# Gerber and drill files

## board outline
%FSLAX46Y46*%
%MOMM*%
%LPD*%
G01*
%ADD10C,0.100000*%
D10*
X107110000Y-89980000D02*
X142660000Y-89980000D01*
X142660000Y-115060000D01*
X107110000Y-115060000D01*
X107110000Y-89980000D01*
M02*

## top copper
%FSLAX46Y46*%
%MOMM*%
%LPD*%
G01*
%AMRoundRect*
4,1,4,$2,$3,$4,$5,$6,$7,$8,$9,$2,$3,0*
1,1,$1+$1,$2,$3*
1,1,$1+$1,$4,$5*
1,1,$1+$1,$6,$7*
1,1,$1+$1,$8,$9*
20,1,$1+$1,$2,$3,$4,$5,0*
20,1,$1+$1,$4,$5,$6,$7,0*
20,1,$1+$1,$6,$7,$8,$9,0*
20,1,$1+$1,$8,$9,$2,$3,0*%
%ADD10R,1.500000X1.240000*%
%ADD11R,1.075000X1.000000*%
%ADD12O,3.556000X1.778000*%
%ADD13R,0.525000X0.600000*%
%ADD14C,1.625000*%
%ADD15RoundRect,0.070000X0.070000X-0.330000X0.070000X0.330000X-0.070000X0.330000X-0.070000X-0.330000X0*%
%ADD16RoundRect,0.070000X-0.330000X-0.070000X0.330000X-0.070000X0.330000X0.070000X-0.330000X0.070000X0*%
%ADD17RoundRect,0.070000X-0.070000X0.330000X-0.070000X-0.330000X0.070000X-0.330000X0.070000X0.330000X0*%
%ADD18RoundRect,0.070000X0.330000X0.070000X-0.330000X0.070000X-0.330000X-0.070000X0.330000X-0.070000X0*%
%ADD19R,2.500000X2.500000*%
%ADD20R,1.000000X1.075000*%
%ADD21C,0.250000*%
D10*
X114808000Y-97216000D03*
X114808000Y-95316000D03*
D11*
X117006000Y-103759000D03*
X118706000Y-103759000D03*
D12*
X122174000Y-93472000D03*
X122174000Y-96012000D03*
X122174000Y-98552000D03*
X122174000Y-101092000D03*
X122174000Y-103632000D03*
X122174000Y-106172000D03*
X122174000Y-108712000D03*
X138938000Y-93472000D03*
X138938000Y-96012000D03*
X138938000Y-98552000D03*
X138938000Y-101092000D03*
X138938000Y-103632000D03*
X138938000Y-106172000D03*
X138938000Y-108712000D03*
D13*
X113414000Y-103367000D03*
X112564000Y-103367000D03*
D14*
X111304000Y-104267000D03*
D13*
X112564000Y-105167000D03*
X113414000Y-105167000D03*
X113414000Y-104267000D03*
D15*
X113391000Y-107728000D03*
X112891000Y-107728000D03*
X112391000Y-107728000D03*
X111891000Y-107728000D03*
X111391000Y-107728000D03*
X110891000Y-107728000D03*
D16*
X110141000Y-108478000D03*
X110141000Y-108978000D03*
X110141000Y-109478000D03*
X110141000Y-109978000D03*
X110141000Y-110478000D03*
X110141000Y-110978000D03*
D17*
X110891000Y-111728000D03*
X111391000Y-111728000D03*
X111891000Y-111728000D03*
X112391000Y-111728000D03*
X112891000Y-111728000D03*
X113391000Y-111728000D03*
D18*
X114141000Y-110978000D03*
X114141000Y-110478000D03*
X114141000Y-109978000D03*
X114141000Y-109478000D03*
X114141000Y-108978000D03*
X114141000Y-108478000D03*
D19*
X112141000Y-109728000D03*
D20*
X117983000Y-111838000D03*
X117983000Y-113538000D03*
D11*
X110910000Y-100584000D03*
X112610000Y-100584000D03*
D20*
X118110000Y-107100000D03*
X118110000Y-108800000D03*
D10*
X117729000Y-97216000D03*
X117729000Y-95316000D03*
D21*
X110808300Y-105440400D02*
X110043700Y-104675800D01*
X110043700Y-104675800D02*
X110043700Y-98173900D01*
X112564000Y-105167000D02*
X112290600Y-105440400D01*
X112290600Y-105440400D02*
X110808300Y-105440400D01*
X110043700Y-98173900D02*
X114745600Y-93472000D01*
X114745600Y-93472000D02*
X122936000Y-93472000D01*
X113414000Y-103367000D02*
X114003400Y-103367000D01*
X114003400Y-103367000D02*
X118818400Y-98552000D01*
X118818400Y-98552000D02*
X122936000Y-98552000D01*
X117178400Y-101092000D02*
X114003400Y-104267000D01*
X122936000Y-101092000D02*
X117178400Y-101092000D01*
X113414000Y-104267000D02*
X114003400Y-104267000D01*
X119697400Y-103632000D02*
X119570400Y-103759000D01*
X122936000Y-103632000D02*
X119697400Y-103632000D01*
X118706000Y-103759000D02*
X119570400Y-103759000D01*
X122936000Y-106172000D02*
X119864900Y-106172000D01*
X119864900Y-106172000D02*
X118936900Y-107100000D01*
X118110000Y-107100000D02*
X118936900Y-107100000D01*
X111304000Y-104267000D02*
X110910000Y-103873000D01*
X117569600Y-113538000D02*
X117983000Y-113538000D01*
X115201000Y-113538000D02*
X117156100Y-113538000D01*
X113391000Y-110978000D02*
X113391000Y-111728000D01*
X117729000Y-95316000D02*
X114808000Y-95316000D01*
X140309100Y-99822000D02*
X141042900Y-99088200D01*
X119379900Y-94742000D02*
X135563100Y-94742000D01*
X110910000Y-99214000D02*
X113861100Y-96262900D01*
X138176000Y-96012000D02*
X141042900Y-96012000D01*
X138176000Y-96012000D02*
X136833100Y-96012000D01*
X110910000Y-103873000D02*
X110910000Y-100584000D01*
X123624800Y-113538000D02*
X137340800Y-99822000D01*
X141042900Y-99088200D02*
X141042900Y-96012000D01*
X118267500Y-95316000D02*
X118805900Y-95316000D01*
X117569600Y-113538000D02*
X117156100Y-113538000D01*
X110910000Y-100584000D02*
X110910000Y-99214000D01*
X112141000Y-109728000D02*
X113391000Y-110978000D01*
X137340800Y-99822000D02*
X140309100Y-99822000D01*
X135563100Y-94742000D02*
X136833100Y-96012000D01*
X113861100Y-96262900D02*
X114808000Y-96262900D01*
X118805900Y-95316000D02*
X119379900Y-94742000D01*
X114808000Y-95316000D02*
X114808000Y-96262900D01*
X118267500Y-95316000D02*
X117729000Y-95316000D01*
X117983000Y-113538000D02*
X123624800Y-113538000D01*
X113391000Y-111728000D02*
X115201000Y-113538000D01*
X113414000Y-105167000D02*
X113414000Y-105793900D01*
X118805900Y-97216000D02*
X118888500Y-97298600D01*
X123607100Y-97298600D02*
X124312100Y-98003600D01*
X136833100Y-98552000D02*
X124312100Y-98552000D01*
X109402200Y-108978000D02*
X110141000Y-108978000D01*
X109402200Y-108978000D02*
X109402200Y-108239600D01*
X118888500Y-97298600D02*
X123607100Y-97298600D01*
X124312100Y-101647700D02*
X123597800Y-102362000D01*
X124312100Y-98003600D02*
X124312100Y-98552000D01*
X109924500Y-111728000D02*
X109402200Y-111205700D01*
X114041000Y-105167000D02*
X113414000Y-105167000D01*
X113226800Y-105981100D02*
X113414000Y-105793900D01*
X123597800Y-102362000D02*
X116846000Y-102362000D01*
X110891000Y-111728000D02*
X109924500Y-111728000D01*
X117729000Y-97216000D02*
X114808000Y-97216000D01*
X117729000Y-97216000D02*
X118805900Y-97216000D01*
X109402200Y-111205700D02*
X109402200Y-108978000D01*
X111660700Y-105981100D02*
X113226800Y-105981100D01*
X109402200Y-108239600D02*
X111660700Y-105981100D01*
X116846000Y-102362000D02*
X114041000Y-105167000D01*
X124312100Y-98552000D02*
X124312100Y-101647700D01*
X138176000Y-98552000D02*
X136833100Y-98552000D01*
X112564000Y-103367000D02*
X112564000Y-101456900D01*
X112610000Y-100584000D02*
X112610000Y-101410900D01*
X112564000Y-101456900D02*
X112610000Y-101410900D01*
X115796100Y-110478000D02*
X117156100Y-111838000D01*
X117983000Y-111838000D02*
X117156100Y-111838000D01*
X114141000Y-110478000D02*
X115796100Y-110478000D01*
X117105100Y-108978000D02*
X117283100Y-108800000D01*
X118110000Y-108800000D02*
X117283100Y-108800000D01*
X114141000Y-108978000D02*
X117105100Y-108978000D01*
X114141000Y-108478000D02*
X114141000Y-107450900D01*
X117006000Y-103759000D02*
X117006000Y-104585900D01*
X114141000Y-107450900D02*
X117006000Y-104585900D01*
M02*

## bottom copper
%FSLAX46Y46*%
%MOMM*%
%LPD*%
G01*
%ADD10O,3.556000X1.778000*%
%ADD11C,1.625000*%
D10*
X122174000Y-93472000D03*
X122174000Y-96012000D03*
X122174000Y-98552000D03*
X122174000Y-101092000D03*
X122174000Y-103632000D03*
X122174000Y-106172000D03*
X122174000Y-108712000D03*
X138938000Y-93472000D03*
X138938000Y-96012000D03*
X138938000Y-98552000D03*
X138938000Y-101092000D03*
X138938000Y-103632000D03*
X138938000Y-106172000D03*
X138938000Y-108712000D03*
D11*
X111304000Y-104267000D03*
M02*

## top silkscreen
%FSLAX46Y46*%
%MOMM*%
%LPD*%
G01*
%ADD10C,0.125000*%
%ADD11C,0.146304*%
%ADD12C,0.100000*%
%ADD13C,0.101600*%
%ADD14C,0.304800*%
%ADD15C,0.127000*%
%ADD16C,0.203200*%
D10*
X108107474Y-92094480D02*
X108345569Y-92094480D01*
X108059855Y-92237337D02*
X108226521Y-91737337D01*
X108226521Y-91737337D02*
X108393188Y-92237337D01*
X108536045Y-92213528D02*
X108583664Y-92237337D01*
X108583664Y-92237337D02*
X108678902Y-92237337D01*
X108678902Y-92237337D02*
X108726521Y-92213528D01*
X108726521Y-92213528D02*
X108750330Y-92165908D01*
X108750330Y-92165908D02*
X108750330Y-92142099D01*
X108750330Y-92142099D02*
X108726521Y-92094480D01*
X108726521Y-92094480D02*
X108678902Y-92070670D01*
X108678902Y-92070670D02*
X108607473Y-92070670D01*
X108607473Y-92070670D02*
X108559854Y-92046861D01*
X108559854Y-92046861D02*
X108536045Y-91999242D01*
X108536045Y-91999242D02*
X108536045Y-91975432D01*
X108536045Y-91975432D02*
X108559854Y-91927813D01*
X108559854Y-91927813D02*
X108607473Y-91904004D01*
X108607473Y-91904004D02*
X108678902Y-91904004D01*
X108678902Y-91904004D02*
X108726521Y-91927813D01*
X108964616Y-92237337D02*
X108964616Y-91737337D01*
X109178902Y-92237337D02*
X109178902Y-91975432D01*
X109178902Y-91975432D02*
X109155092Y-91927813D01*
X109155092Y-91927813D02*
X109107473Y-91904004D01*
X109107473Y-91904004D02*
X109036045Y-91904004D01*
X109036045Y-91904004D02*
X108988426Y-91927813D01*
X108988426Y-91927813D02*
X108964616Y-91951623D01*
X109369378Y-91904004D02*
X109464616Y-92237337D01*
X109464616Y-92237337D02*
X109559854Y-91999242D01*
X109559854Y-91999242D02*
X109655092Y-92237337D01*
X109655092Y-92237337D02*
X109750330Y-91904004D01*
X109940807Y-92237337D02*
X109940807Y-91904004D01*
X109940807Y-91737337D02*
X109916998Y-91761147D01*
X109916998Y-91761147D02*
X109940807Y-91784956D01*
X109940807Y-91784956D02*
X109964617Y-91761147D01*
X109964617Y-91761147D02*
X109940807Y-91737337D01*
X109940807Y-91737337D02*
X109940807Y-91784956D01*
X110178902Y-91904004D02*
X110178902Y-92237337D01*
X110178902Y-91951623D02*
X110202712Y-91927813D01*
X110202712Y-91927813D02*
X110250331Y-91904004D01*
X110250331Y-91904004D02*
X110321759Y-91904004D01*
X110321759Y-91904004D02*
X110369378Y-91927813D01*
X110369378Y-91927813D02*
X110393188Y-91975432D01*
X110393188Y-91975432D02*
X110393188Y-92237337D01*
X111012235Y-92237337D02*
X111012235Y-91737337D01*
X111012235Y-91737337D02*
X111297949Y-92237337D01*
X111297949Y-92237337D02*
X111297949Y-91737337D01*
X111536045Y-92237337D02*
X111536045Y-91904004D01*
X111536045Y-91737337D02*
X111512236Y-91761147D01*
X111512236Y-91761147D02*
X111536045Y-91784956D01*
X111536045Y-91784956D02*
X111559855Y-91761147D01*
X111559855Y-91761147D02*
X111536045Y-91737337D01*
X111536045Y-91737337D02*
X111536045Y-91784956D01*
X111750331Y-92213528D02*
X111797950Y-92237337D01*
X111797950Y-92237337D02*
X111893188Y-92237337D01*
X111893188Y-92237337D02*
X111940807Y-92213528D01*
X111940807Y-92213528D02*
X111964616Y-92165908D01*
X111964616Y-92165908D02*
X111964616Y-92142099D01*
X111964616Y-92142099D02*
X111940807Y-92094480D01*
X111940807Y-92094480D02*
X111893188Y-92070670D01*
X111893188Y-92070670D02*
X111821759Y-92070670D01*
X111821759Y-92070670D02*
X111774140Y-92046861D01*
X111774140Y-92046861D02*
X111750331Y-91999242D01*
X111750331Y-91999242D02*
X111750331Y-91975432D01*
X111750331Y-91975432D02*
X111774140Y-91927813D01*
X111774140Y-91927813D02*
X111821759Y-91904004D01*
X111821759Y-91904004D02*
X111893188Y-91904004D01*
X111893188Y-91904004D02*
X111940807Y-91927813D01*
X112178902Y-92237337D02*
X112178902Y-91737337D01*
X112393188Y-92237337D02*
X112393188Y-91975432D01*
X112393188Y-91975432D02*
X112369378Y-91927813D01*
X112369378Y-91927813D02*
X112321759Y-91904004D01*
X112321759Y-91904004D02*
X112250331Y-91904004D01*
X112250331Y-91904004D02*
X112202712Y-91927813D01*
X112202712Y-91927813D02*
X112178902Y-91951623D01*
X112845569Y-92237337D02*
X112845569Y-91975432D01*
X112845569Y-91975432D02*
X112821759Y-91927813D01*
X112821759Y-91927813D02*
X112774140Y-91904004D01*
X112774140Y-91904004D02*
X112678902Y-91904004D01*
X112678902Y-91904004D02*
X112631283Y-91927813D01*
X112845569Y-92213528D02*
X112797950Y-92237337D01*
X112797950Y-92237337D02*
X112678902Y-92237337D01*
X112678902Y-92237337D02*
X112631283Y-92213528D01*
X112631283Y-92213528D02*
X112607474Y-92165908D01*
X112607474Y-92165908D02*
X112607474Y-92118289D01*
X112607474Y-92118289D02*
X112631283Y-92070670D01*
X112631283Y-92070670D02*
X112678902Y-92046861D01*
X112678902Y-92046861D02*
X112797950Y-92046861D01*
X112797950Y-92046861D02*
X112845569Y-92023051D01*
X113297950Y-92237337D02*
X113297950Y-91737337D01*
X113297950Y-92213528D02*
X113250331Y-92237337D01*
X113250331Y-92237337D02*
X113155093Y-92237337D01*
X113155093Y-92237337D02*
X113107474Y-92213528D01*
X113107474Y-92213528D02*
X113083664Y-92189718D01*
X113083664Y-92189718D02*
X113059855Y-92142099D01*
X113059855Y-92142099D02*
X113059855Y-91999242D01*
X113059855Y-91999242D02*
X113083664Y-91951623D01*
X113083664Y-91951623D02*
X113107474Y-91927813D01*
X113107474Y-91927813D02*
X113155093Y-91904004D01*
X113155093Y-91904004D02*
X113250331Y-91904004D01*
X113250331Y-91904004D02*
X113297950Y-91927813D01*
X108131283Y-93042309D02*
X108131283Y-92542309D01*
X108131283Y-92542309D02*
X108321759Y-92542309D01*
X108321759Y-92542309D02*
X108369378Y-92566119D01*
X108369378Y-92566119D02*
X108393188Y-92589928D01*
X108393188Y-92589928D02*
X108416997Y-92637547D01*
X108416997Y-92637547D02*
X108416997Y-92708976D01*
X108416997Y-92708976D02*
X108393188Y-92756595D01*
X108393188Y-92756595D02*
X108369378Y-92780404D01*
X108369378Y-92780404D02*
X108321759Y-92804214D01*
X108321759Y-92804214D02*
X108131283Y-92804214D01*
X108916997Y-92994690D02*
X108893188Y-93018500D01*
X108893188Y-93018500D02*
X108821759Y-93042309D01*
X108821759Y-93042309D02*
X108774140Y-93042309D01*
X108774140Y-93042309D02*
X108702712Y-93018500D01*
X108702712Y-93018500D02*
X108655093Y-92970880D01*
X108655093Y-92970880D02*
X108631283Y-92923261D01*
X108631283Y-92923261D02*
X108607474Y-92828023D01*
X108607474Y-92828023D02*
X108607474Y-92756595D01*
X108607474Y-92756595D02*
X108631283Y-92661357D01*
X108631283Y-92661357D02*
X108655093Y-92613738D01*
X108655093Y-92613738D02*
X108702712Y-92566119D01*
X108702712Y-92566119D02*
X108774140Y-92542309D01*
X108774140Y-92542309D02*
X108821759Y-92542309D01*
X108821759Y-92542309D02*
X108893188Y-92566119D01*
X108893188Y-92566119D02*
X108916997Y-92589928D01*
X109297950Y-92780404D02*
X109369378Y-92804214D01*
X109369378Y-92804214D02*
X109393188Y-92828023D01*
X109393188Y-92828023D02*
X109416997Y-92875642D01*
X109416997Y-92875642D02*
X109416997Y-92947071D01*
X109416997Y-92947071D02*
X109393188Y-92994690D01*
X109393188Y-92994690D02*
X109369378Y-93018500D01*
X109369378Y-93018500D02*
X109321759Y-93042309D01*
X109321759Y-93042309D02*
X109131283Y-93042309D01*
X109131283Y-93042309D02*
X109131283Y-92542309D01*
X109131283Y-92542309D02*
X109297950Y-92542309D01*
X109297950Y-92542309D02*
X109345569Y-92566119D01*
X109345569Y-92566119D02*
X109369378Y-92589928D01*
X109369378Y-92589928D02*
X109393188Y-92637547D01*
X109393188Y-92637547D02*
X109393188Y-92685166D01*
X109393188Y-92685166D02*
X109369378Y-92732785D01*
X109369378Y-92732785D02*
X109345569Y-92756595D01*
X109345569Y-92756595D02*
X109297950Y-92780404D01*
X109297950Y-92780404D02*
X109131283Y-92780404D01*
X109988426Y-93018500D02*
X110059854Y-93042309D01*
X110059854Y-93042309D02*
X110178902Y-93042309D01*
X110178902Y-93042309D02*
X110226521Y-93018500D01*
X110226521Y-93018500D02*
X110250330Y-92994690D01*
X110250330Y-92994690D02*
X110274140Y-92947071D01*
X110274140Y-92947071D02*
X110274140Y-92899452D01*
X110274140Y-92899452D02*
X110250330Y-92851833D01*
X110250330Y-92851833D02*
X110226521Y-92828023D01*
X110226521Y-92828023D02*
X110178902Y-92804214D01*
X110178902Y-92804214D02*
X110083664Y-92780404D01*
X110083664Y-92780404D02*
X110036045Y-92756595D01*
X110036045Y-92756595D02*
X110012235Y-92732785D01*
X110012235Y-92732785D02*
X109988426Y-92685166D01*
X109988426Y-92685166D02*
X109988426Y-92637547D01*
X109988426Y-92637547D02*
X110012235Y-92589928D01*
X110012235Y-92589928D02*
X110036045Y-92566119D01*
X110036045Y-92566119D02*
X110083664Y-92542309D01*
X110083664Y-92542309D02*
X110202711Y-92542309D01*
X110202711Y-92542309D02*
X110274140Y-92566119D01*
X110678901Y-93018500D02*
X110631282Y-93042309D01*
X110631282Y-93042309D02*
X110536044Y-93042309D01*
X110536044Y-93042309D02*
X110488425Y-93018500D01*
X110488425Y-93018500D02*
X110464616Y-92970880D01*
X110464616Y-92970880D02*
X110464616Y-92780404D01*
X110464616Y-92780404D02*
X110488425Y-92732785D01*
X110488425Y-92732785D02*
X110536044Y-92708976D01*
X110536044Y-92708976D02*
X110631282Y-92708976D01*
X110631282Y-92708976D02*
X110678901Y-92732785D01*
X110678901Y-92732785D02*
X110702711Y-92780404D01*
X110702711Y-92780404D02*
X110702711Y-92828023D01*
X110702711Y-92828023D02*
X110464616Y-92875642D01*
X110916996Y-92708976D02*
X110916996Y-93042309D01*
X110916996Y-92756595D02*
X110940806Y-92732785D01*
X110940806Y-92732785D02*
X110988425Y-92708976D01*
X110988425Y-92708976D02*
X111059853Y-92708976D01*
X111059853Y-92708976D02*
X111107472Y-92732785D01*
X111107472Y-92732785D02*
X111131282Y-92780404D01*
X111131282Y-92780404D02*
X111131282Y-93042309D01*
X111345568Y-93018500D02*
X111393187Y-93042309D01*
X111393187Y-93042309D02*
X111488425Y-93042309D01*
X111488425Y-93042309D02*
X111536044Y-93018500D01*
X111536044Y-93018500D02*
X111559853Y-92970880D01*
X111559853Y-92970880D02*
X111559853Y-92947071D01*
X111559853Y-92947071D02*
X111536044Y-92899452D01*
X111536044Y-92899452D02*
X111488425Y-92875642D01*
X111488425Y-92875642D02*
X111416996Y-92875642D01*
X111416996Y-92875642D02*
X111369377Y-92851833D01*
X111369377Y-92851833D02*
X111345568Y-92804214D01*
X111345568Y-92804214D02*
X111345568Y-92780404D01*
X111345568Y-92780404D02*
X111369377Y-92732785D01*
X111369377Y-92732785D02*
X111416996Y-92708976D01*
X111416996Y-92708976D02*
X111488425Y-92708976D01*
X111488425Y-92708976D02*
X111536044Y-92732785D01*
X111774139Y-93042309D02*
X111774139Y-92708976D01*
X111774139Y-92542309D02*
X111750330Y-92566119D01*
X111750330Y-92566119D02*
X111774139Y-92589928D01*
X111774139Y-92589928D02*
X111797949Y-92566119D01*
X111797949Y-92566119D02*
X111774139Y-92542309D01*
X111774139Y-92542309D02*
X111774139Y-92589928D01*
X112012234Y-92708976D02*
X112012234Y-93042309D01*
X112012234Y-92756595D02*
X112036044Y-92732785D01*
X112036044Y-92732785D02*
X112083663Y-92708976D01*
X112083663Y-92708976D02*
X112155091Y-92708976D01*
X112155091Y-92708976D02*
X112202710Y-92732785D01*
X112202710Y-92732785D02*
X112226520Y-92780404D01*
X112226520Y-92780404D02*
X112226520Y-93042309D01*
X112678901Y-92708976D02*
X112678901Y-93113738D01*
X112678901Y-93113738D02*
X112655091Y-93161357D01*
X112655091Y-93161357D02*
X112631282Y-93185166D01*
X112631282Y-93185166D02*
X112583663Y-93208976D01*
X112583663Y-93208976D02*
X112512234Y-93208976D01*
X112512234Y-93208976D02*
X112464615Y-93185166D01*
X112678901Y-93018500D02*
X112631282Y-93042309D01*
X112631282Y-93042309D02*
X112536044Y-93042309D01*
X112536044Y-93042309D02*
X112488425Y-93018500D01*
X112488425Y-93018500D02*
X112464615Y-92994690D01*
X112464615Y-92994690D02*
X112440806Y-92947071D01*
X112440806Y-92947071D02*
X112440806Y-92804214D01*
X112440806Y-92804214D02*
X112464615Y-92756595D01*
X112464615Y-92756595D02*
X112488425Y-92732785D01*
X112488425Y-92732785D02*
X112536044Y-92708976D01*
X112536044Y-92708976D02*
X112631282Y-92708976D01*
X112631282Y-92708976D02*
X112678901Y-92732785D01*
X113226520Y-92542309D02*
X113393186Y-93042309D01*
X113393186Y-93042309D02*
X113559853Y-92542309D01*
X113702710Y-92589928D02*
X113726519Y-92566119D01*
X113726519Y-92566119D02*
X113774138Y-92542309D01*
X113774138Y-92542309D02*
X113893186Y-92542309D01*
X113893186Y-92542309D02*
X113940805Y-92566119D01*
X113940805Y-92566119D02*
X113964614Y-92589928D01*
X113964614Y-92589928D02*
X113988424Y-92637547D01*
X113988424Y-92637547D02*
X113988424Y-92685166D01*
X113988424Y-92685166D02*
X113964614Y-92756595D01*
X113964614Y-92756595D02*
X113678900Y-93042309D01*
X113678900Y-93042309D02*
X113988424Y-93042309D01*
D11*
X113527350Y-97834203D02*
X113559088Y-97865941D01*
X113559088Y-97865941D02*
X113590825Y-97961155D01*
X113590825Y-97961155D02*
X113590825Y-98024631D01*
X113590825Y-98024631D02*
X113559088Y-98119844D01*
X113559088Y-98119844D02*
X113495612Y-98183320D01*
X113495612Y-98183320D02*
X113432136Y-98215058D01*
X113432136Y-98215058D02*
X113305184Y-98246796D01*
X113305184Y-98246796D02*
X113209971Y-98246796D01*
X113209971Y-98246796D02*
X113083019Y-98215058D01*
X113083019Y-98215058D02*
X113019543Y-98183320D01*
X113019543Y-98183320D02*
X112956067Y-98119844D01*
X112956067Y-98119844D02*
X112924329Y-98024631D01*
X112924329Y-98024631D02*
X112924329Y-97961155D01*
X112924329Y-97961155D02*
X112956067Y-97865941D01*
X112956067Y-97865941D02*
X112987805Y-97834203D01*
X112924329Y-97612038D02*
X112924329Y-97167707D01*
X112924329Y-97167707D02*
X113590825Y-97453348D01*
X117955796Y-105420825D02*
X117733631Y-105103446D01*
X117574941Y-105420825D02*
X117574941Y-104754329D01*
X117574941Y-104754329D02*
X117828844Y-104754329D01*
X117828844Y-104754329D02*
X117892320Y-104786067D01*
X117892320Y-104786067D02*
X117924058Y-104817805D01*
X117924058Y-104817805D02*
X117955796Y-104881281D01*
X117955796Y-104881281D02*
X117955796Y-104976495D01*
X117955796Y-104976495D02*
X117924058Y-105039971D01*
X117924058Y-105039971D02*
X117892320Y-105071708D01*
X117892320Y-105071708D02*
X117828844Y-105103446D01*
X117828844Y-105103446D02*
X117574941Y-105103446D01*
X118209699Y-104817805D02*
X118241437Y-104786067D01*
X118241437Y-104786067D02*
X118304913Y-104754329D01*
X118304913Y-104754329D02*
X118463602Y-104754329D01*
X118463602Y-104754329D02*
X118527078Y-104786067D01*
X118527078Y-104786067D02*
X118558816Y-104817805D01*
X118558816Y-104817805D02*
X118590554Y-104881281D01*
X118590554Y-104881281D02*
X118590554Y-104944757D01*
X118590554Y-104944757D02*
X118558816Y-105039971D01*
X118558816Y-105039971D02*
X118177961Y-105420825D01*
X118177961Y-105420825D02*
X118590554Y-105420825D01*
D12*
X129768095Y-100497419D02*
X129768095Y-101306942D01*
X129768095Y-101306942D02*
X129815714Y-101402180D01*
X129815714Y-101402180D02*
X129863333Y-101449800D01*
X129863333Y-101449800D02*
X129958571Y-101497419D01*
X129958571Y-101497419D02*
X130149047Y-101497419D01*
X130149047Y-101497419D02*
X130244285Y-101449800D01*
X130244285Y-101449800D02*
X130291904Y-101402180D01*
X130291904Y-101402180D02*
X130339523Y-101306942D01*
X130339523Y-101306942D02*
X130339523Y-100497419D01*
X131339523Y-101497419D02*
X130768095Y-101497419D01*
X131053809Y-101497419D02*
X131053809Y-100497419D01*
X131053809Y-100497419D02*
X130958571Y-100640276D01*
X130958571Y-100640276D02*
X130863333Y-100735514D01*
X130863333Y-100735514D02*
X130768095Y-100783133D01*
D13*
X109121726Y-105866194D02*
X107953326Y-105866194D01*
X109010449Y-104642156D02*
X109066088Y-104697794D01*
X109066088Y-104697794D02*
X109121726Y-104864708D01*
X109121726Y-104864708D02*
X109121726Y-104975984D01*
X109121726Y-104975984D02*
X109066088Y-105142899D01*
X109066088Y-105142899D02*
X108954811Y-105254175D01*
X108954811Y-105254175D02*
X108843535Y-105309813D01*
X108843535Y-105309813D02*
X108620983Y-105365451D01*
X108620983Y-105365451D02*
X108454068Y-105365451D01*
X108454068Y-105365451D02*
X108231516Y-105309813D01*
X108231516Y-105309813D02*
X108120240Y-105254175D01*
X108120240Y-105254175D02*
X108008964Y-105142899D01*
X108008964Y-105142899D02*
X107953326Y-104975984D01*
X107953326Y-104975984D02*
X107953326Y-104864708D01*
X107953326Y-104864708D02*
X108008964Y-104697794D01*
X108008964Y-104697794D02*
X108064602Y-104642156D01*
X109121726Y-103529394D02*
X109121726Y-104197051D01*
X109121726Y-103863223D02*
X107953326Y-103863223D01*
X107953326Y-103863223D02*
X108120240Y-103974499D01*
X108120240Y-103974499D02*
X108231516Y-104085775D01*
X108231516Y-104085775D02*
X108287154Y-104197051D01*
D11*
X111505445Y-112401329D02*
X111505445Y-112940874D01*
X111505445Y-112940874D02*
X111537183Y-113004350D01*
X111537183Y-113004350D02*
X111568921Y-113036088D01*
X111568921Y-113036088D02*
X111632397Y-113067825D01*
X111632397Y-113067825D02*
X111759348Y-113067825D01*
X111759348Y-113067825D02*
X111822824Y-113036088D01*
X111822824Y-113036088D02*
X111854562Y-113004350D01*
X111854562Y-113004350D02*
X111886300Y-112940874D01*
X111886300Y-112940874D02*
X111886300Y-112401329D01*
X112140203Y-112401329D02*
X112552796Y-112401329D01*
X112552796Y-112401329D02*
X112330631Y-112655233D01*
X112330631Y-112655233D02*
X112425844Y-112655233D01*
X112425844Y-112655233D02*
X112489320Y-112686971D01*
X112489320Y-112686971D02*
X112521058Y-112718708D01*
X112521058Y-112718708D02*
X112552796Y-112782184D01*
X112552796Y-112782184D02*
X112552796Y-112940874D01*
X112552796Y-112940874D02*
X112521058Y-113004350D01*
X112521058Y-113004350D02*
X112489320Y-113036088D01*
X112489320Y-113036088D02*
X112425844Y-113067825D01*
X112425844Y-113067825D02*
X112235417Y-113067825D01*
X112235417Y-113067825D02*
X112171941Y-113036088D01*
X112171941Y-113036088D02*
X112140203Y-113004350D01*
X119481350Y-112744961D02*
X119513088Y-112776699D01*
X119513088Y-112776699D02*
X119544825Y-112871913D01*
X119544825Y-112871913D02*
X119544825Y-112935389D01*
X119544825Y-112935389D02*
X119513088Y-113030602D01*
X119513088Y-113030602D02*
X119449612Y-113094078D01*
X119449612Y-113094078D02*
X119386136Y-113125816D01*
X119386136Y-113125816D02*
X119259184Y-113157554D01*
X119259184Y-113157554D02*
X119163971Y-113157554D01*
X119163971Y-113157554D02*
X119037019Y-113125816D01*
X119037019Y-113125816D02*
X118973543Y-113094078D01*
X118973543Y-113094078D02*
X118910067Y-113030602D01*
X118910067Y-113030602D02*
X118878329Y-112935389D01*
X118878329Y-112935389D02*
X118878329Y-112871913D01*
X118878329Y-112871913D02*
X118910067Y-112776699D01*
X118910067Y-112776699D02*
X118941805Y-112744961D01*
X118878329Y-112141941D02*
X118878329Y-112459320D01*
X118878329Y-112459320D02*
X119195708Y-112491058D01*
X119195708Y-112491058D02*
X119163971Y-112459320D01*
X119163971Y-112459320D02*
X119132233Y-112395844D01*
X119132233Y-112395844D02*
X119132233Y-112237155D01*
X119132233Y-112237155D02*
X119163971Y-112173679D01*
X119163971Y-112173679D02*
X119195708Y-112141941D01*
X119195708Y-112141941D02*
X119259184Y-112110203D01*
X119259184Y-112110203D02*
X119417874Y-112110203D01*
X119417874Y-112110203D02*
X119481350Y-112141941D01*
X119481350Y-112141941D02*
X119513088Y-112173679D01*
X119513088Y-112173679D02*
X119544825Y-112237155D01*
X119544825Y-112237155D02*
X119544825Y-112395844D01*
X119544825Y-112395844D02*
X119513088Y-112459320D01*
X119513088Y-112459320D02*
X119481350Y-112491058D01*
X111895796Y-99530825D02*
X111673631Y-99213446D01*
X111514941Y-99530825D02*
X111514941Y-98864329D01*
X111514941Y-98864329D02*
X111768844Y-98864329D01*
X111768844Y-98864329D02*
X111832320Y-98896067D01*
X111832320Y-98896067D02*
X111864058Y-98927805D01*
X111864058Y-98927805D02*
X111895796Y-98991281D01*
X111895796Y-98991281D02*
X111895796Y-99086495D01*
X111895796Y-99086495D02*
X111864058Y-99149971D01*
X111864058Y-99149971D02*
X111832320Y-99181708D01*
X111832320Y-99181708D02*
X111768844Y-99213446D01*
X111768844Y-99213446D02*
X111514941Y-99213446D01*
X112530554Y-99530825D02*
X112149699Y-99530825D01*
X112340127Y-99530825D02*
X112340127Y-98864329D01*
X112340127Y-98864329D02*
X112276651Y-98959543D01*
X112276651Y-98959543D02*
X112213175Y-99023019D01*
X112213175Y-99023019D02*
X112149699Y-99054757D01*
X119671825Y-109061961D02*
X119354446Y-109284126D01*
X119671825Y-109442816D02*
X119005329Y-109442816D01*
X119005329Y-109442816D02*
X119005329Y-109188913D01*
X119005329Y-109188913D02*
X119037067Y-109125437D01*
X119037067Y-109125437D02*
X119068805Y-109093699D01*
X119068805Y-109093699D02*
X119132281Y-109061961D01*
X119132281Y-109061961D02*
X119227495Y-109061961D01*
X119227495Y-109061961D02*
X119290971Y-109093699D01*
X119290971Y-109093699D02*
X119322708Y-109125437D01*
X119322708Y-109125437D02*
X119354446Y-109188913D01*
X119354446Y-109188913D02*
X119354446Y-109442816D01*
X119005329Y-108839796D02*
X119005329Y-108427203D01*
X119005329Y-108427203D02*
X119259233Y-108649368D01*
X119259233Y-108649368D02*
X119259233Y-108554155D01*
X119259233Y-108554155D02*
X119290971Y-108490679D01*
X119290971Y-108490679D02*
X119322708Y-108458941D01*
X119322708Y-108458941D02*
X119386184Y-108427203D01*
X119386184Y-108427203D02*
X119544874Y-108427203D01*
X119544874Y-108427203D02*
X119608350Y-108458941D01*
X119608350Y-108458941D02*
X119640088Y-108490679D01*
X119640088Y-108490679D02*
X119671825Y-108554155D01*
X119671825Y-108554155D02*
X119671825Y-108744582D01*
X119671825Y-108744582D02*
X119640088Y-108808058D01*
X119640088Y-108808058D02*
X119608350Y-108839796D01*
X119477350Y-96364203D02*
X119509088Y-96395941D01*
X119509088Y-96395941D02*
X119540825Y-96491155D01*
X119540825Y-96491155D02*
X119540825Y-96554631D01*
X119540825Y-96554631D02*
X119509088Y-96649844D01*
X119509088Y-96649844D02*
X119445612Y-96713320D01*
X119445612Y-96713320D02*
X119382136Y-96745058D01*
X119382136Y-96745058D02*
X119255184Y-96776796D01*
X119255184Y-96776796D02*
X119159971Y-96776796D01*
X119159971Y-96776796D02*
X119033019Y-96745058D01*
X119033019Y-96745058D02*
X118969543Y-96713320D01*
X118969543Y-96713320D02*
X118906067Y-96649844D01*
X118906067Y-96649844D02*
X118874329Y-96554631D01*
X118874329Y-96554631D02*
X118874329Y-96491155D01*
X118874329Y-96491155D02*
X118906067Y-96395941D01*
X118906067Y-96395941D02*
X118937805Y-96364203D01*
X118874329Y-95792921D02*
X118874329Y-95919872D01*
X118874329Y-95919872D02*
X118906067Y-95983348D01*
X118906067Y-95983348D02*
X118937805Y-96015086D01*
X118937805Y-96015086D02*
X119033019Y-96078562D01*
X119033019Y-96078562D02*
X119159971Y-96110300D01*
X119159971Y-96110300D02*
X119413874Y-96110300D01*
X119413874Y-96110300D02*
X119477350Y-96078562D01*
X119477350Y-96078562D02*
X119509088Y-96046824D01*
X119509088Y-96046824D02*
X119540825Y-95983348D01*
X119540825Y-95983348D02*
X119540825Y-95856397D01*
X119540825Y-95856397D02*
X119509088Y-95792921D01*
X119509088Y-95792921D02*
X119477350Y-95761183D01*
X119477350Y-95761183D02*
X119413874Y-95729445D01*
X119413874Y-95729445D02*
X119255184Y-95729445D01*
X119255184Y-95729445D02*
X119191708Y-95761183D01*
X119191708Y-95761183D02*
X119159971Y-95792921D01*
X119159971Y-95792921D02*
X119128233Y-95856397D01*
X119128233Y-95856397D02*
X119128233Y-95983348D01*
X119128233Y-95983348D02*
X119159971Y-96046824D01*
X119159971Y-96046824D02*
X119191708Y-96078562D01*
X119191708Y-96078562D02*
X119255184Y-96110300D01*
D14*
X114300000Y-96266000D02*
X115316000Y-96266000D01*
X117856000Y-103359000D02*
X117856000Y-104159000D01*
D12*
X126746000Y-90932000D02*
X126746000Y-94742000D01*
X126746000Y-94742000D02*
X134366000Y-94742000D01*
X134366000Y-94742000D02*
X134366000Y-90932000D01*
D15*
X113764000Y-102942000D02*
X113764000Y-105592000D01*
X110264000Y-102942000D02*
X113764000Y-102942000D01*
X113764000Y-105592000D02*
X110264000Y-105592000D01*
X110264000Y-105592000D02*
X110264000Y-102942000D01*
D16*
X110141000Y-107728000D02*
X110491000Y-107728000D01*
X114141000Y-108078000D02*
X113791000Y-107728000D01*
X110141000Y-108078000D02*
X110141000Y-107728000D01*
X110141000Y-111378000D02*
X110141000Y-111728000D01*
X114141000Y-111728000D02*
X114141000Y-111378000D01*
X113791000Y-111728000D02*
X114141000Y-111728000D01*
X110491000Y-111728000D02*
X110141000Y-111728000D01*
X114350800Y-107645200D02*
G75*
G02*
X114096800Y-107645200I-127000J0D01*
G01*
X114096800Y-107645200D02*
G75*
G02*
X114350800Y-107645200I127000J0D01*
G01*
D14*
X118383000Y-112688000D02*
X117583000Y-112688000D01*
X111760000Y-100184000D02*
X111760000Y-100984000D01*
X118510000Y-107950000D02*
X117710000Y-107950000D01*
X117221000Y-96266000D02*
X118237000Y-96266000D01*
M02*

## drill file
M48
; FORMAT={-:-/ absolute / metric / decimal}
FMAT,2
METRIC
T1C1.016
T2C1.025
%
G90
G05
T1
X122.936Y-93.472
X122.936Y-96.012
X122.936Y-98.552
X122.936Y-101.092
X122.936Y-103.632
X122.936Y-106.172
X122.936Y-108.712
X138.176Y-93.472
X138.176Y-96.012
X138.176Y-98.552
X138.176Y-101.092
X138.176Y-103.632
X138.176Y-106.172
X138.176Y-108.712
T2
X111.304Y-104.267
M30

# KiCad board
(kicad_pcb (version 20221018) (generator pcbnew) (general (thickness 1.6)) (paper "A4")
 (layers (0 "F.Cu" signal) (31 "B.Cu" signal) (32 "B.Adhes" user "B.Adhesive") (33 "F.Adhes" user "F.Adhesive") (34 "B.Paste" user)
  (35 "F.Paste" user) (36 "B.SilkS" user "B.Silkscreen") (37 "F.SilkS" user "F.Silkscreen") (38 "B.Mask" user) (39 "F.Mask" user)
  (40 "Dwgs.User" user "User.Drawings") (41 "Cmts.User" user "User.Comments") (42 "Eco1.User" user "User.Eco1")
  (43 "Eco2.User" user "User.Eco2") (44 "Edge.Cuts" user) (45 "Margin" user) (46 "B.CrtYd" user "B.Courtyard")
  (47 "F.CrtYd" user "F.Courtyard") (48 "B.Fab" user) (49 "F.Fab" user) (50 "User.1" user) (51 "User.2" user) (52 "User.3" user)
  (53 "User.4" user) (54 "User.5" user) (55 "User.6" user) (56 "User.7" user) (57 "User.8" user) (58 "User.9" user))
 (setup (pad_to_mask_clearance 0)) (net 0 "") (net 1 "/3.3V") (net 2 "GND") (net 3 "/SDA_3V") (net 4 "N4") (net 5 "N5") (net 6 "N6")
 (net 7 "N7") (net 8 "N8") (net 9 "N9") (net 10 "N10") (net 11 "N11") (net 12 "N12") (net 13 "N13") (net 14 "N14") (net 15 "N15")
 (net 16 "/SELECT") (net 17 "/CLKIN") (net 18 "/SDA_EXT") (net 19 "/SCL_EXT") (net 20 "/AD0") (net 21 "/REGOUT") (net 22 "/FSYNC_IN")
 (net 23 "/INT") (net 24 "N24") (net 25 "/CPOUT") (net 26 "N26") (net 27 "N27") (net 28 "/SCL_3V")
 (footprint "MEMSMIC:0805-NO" (layer "F.Cu") (at 114.808 96.266 90)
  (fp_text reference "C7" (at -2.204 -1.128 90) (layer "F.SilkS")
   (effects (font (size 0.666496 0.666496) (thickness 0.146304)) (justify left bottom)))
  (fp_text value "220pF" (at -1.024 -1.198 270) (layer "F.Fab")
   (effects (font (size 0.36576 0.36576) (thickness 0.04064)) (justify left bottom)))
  (fp_line (start 0 -0.508) (end 0 0.508) (stroke (width 0.3048) (type solid)) (layer "F.SilkS"))
  (pad "1" smd rect (at -0.95 0 90) (size 1.24 1.5) (layers "F.Cu" "F.Paste" "F.Mask") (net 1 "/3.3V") (solder_mask_margin 0.0508)
   (thermal_bridge_angle 0))
  (pad "2" smd rect (at 0.95 0 90) (size 1.24 1.5) (layers "F.Cu" "F.Paste" "F.Mask") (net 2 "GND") (solder_mask_margin 0.0508)
   (thermal_bridge_angle 0)))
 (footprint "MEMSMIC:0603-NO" (layer "F.Cu") (at 117.856 103.759)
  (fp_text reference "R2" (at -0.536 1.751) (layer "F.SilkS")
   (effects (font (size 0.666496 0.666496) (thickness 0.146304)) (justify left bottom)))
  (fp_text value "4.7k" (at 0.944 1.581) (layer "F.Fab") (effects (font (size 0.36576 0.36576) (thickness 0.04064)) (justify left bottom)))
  (fp_line (start 0 -0.4) (end 0 0.4) (stroke (width 0.3048) (type solid)) (layer "F.SilkS"))
  (pad "1" smd rect (at -0.85 0) (size 1.075 1) (layers "F.Cu" "F.Paste" "F.Mask") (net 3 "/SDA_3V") (solder_mask_margin 0.0508)
   (thermal_bridge_angle 0))
  (pad "2" smd rect (at 0.85 0) (size 1.075 1) (layers "F.Cu" "F.Paste" "F.Mask") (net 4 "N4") (solder_mask_margin 0.0508)
   (thermal_bridge_angle 0)))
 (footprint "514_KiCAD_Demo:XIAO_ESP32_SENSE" (layer "F.Cu") (at 130.556 101.092)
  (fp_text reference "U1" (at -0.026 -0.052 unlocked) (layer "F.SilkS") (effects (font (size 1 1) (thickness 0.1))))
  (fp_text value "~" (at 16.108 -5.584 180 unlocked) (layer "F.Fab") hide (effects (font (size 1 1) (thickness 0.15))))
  (fp_line (start -3.81 -10.16) (end -3.81 -6.35) (stroke (width 0.1) (type default)) (layer "F.SilkS"))
  (fp_line (start -3.81 -6.35) (end 3.81 -6.35) (stroke (width 0.1) (type default)) (layer "F.SilkS"))
  (fp_line (start 3.81 -6.35) (end 3.81 -10.16) (stroke (width 0.1) (type default)) (layer "F.SilkS"))
  (pad "1" thru_hole oval (at -7.62 -7.62) (size 3.556 1.778) (drill 1.016 (offset -0.762 0)) (layers "*.Cu" "*.Mask") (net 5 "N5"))
  (pad "2" thru_hole oval (at -7.62 -5.08) (size 3.556 1.778) (drill 1.016 (offset -0.762 0)) (layers "*.Cu" "*.Mask") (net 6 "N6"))
  (pad "3" thru_hole oval (at -7.62 -2.54) (size 3.556 1.778) (drill 1.016 (offset -0.762 0)) (layers "*.Cu" "*.Mask") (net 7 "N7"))
  (pad "4" thru_hole oval (at -7.62 0) (size 3.556 1.778) (drill 1.016 (offset -0.762 0)) (layers "*.Cu" "*.Mask") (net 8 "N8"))
  (pad "5" thru_hole oval (at -7.62 2.54) (size 3.556 1.778) (drill 1.016 (offset -0.762 0)) (layers "*.Cu" "*.Mask") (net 4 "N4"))
  (pad "6" thru_hole oval (at -7.62 5.08) (size 3.556 1.778) (drill 1.016 (offset -0.762 0)) (layers "*.Cu" "*.Mask") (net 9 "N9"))
  (pad "7" thru_hole oval (at -7.62 7.62) (size 3.556 1.778) (drill 1.016 (offset -0.762 0)) (layers "*.Cu" "*.Mask") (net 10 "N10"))
  (pad "8" thru_hole oval (at 7.62 -7.62) (size 3.556 1.778) (drill 1.016 (offset 0.762 0)) (layers "*.Cu" "*.Mask") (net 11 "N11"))
  (pad "9" thru_hole oval (at 7.62 -5.08) (size 3.556 1.778) (drill 1.016 (offset 0.762 0)) (layers "*.Cu" "*.Mask") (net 2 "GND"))
  (pad "10" thru_hole oval (at 7.62 -2.54) (size 3.556 1.778) (drill 1.016 (offset 0.762 0)) (layers "*.Cu" "*.Mask") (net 1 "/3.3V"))
  (pad "11" thru_hole oval (at 7.62 0) (size 3.556 1.778) (drill 1.016 (offset 0.762 0)) (layers "*.Cu" "*.Mask") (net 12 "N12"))
  (pad "12" thru_hole oval (at 7.62 2.54) (size 3.556 1.778) (drill 1.016 (offset 0.762 0)) (layers "*.Cu" "*.Mask") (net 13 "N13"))
  (pad "13" thru_hole oval (at 7.62 5.08) (size 3.556 1.778) (drill 1.016 (offset 0.762 0)) (layers "*.Cu" "*.Mask") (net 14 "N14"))
  (pad "14" thru_hole oval (at 7.62 7.62) (size 3.556 1.778) (drill 1.016 (offset 0.762 0)) (layers "*.Cu" "*.Mask") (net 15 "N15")))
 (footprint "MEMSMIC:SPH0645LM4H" (layer "F.Cu") (at 112.014 104.267 -90)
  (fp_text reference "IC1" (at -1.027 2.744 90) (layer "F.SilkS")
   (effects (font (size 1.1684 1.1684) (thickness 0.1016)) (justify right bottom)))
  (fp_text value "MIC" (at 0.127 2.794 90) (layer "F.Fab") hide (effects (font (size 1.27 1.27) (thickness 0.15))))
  (fp_line (start -1.325 -1.75) (end 1.325 -1.75) (stroke (width 0.127) (type solid)) (layer "F.SilkS"))
  (fp_line (start -1.325 1.75) (end -1.325 -1.75) (stroke (width 0.127) (type solid)) (layer "F.SilkS"))
  (fp_line (start 1.325 -1.75) (end 1.325 1.75) (stroke (width 0.127) (type solid)) (layer "F.SilkS"))
  (fp_line (start 1.325 1.75) (end -1.325 1.75) (stroke (width 0.127) (type solid)) (layer "F.SilkS"))
  (pad "1" smd rect (at -0.9 -1.4 270) (size 0.6 0.525) (layers "F.Cu" "F.Paste" "F.Mask") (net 7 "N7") (solder_mask_margin 0.0508)
   (thermal_bridge_angle 0))
  (pad "2" smd rect (at -0.9 -0.55 270) (size 0.6 0.525) (layers "F.Cu" "F.Paste" "F.Mask") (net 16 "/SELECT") (solder_mask_margin 0.0508)
   (thermal_bridge_angle 0))
  (pad "3" thru_hole circle (at 0 0.71 270) (size 1.625 1.625) (drill 1.025) (layers "*.Cu" "*.Mask") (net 2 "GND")
   (solder_mask_margin 0.0508) (thermal_bridge_angle 0))
  (pad "4" smd rect (at 0.9 -0.55 270) (size 0.6 0.525) (layers "F.Cu" "F.Paste" "F.Mask") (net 5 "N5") (solder_mask_margin 0.0508)
   (thermal_bridge_angle 0))
  (pad "5" smd rect (at 0.9 -1.4 270) (size 0.6 0.525) (layers "F.Cu" "F.Paste" "F.Mask") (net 1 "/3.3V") (solder_mask_margin 0.0508)
   (thermal_bridge_angle 0))
  (pad "6" smd rect (at 0 -1.4 270) (size 0.6 0.525) (layers "F.Cu" "F.Paste" "F.Mask") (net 8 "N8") (solder_mask_margin 0.0508)
   (thermal_bridge_angle 0)))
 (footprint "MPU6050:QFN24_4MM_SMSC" (layer "F.Cu") (at 112.141 109.728 -90)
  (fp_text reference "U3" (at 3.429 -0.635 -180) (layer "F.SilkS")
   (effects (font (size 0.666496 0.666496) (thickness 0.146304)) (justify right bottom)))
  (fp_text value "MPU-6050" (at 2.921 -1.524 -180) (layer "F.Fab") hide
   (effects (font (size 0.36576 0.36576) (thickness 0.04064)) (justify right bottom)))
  (fp_line (start -2 2) (end -2 1.65) (stroke (width 0.2032) (type solid)) (layer "F.SilkS"))
  (fp_line (start -1.65 -2) (end -2 -1.65) (stroke (width 0.2032) (type solid)) (layer "F.SilkS"))
  (fp_line (start -1.65 2) (end -2 2) (stroke (width 0.2032) (type solid)) (layer "F.SilkS"))
  (fp_line (start 1.65 2) (end 2 2) (stroke (width 0.2032) (type solid)) (layer "F.SilkS"))
  (fp_line (start 2 -2) (end 1.65 -2) (stroke (width 0.2032) (type solid)) (layer "F.SilkS"))
  (fp_line (start 2 -1.65) (end 2 -2) (stroke (width 0.2032) (type solid)) (layer "F.SilkS"))
  (fp_line (start 2 1.65) (end 2 2) (stroke (width 0.2032) (type solid)) (layer "F.SilkS"))
  (fp_circle (center -2.0828 -2.0828) (end -1.9558 -2.0828) (stroke (width 0.2032) (type solid)) (fill none) (layer "F.SilkS"))
  (pad "1" smd roundrect (at -2 -1.25 90) (size 0.8 0.28) (layers "F.Cu" "F.Paste" "F.Mask") (roundrect_rratio 0.25) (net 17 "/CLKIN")
   (solder_mask_margin 0.0508) (thermal_bridge_angle 0))
  (pad "2" smd roundrect (at -2 -0.75 90) (size 0.8 0.28) (layers "F.Cu" "F.Paste" "F.Mask") (roundrect_rratio 0.25)
   (solder_mask_margin 0.0508) (thermal_bridge_angle 0))
  (pad "3" smd roundrect (at -2 -0.25 90) (size 0.8 0.28) (layers "F.Cu" "F.Paste" "F.Mask") (roundrect_rratio 0.25)
   (solder_mask_margin 0.0508) (thermal_bridge_angle 0))
  (pad "4" smd roundrect (at -2 0.25 90) (size 0.8 0.28) (layers "F.Cu" "F.Paste" "F.Mask") (roundrect_rratio 0.25)
   (solder_mask_margin 0.0508) (thermal_bridge_angle 0))
  (pad "5" smd roundrect (at -2 0.75 90) (size 0.8 0.28) (layers "F.Cu" "F.Paste" "F.Mask") (roundrect_rratio 0.25)
   (solder_mask_margin 0.0508) (thermal_bridge_angle 0))
  (pad "6" smd roundrect (at -2 1.25 90) (size 0.8 0.28) (layers "F.Cu" "F.Paste" "F.Mask") (roundrect_rratio 0.25) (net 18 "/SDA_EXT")
   (solder_mask_margin 0.0508) (thermal_bridge_angle 0))
  (pad "7" smd roundrect (at -1.25 2) (size 0.8 0.28) (layers "F.Cu" "F.Paste" "F.Mask") (roundrect_rratio 0.25) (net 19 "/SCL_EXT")
   (solder_mask_margin 0.0508) (thermal_bridge_angle 0))
  (pad "8" smd roundrect (at -0.75 2) (size 0.8 0.28) (layers "F.Cu" "F.Paste" "F.Mask") (roundrect_rratio 0.25) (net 1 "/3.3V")
   (solder_mask_margin 0.0508) (thermal_bridge_angle 0))
  (pad "9" smd roundrect (at -0.25 2) (size 0.8 0.28) (layers "F.Cu" "F.Paste" "F.Mask") (roundrect_rratio 0.25) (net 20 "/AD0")
   (solder_mask_margin 0.0508) (thermal_bridge_angle 0))
  (pad "10" smd roundrect (at 0.25 2) (size 0.8 0.28) (layers "F.Cu" "F.Paste" "F.Mask") (roundrect_rratio 0.25) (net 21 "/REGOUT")
   (solder_mask_margin 0.0508) (thermal_bridge_angle 0))
  (pad "11" smd roundrect (at 0.75 2) (size 0.8 0.28) (layers "F.Cu" "F.Paste" "F.Mask") (roundrect_rratio 0.25) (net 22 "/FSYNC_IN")
   (solder_mask_margin 0.0508) (thermal_bridge_angle 0))
  (pad "12" smd roundrect (at 1.25 2) (size 0.8 0.28) (layers "F.Cu" "F.Paste" "F.Mask") (roundrect_rratio 0.25) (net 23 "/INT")
   (solder_mask_margin 0.0508) (thermal_bridge_angle 0))
  (pad "13" smd roundrect (at 2 1.25 270) (size 0.8 0.28) (layers "F.Cu" "F.Paste" "F.Mask") (roundrect_rratio 0.25) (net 1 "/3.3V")
   (solder_mask_margin 0.0508) (thermal_bridge_angle 0))
  (pad "14" smd roundrect (at 2 0.75 270) (size 0.8 0.28) (layers "F.Cu" "F.Paste" "F.Mask") (roundrect_rratio 0.25)
   (solder_mask_margin 0.0508) (thermal_bridge_angle 0))
  (pad "15" smd roundrect (at 2 0.25 270) (size 0.8 0.28) (layers "F.Cu" "F.Paste" "F.Mask") (roundrect_rratio 0.25)
   (solder_mask_margin 0.0508) (thermal_bridge_angle 0))
  (pad "16" smd roundrect (at 2 -0.25 270) (size 0.8 0.28) (layers "F.Cu" "F.Paste" "F.Mask") (roundrect_rratio 0.25)
   (solder_mask_margin 0.0508) (thermal_bridge_angle 0))
  (pad "17" smd roundrect (at 2 -0.75 270) (size 0.8 0.28) (layers "F.Cu" "F.Paste" "F.Mask") (roundrect_rratio 0.25)
   (solder_mask_margin 0.0508) (thermal_bridge_angle 0))
  (pad "18" smd roundrect (at 2 -1.25 270) (size 0.8 0.28) (layers "F.Cu" "F.Paste" "F.Mask") (roundrect_rratio 0.25) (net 2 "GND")
   (solder_mask_margin 0.0508) (thermal_bridge_angle 0))
  (pad "19" smd roundrect (at 1.25 -2 180) (size 0.8 0.28) (layers "F.Cu" "F.Paste" "F.Mask") (roundrect_rratio 0.25) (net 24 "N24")
   (solder_mask_margin 0.0508) (thermal_bridge_angle 0))
  (pad "20" smd roundrect (at 0.75 -2 180) (size 0.8 0.28) (layers "F.Cu" "F.Paste" "F.Mask") (roundrect_rratio 0.25) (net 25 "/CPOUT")
   (solder_mask_margin 0.0508) (thermal_bridge_angle 0))
  (pad "21" smd roundrect (at 0.25 -2 180) (size 0.8 0.28) (layers "F.Cu" "F.Paste" "F.Mask") (roundrect_rratio 0.25) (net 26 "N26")
   (solder_mask_margin 0.0508) (thermal_bridge_angle 0))
  (pad "22" smd roundrect (at -0.25 -2 180) (size 0.8 0.28) (layers "F.Cu" "F.Paste" "F.Mask") (roundrect_rratio 0.25) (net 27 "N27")
   (solder_mask_margin 0.0508) (thermal_bridge_angle 0))
  (pad "23" smd roundrect (at -0.75 -2 180) (size 0.8 0.28) (layers "F.Cu" "F.Paste" "F.Mask") (roundrect_rratio 0.25) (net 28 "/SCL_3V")
   (solder_mask_margin 0.0508) (thermal_bridge_angle 0))
  (pad "24" smd roundrect (at -1.25 -2 180) (size 0.8 0.28) (layers "F.Cu" "F.Paste" "F.Mask") (roundrect_rratio 0.25) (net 3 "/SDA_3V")
   (solder_mask_margin 0.0508) (thermal_bridge_angle 0))
  (pad "THERM" smd rect (at 0 0 270) (size 2.5 2.5) (layers "F.Cu" "F.Mask") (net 2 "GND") (solder_mask_margin 0.0508)
   (thermal_bridge_angle 0)))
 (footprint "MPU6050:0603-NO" (layer "F.Cu") (at 117.983 112.688 -90)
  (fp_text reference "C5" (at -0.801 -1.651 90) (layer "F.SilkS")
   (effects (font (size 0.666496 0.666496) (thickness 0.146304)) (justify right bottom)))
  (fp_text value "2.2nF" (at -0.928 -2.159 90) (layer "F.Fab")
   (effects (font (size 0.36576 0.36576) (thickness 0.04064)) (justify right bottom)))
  (fp_line (start 0 -0.4) (end 0 0.4) (stroke (width 0.3048) (type solid)) (layer "F.SilkS"))
  (pad "1" smd rect (at -0.85 0 270) (size 1.075 1) (layers "F.Cu" "F.Paste" "F.Mask") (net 25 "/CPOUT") (solder_mask_margin 0.0508)
   (thermal_bridge_angle 0))
  (pad "2" smd rect (at 0.85 0 270) (size 1.075 1) (layers "F.Cu" "F.Paste" "F.Mask") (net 2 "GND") (solder_mask_margin 0.0508)
   (thermal_bridge_angle 0)))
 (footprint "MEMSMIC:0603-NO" (layer "F.Cu") (at 111.76 100.584)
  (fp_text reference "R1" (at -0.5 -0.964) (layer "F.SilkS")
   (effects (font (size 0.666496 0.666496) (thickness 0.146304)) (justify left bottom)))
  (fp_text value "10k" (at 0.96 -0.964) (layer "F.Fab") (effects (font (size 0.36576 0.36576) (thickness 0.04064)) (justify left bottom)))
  (fp_line (start 0 -0.4) (end 0 0.4) (stroke (width 0.3048) (type solid)) (layer "F.SilkS"))
  (pad "1" smd rect (at -0.85 0) (size 1.075 1) (layers "F.Cu" "F.Paste" "F.Mask") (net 2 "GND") (solder_mask_margin 0.0508)
   (thermal_bridge_angle 0))
  (pad "2" smd rect (at 0.85 0) (size 1.075 1) (layers "F.Cu" "F.Paste" "F.Mask") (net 16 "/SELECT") (solder_mask_margin 0.0508)
   (thermal_bridge_angle 0)))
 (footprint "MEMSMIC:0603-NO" (layer "F.Cu") (at 118.11 107.95 -90)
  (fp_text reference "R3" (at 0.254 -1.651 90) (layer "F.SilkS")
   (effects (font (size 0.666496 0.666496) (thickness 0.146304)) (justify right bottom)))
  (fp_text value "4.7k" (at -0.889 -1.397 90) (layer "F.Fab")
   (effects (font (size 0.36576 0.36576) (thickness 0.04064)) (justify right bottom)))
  (fp_line (start 0 -0.4) (end 0 0.4) (stroke (width 0.3048) (type solid)) (layer "F.SilkS"))
  (pad "1" smd rect (at -0.85 0 270) (size 1.075 1) (layers "F.Cu" "F.Paste" "F.Mask") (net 9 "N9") (solder_mask_margin 0.0508)
   (thermal_bridge_angle 0))
  (pad "2" smd rect (at 0.85 0 270) (size 1.075 1) (layers "F.Cu" "F.Paste" "F.Mask") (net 28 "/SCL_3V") (solder_mask_margin 0.0508)
   (thermal_bridge_angle 0)))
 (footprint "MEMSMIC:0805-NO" (layer "F.Cu") (at 117.729 96.266 90)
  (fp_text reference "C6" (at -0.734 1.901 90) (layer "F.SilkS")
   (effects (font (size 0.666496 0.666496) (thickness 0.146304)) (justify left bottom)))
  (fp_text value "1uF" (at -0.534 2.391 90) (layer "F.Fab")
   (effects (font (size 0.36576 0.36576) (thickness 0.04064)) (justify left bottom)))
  (fp_line (start 0 -0.508) (end 0 0.508) (stroke (width 0.3048) (type solid)) (layer "F.SilkS"))
  (pad "1" smd rect (at -0.95 0 90) (size 1.24 1.5) (layers "F.Cu" "F.Paste" "F.Mask") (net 1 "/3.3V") (solder_mask_margin 0.0508)
   (thermal_bridge_angle 0))
  (pad "2" smd rect (at 0.95 0 90) (size 1.24 1.5) (layers "F.Cu" "F.Paste" "F.Mask") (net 2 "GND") (solder_mask_margin 0.0508)
   (thermal_bridge_angle 0)))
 (gr_rect (start 107.11 89.98) (end 142.66 115.06) (stroke (width 0.1) (type default)) (fill none) (layer "Edge.Cuts"))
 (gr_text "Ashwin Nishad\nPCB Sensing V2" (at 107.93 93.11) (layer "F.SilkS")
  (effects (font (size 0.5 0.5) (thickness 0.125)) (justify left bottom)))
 (segment (start 110.8083 105.4404) (end 110.0437 104.6758) (width 0.25) (layer "F.Cu") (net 5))
 (segment (start 110.0437 104.6758) (end 110.0437 98.1739) (width 0.25) (layer "F.Cu") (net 5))
 (segment (start 112.564 105.167) (end 112.2906 105.4404) (width 0.25) (layer "F.Cu") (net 5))
 (segment (start 112.2906 105.4404) (end 110.8083 105.4404) (width 0.25) (layer "F.Cu") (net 5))
 (segment (start 110.0437 98.1739) (end 114.7456 93.472) (width 0.25) (layer "F.Cu") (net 5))
 (segment (start 114.7456 93.472) (end 122.936 93.472) (width 0.25) (layer "F.Cu") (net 5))
 (segment (start 113.414 103.367) (end 114.0034 103.367) (width 0.25) (layer "F.Cu") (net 7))
 (segment (start 114.0034 103.367) (end 118.8184 98.552) (width 0.25) (layer "F.Cu") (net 7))
 (segment (start 118.8184 98.552) (end 122.936 98.552) (width 0.25) (layer "F.Cu") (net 7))
 (segment (start 117.1784 101.092) (end 114.0034 104.267) (width 0.25) (layer "F.Cu") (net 8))
 (segment (start 122.936 101.092) (end 117.1784 101.092) (width 0.25) (layer "F.Cu") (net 8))
 (segment (start 113.414 104.267) (end 114.0034 104.267) (width 0.25) (layer "F.Cu") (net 8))
 (segment (start 119.6974 103.632) (end 119.5704 103.759) (width 0.25) (layer "F.Cu") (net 4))
 (segment (start 122.936 103.632) (end 119.6974 103.632) (width 0.25) (layer "F.Cu") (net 4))
 (segment (start 118.706 103.759) (end 119.5704 103.759) (width 0.25) (layer "F.Cu") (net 4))
 (segment (start 122.936 106.172) (end 119.8649 106.172) (width 0.25) (layer "F.Cu") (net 9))
 (segment (start 119.8649 106.172) (end 118.9369 107.1) (width 0.25) (layer "F.Cu") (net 9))
 (segment (start 118.11 107.1) (end 118.9369 107.1) (width 0.25) (layer "F.Cu") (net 9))
 (segment (start 111.304 104.267) (end 110.91 103.873) (width 0.25) (layer "F.Cu") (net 2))
 (segment (start 117.5696 113.538) (end 117.983 113.538) (width 0.25) (layer "F.Cu") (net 2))
 (segment (start 115.201 113.538) (end 117.1561 113.538) (width 0.25) (layer "F.Cu") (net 2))
 (segment (start 113.391 110.978) (end 113.391 111.728) (width 0.25) (layer "F.Cu") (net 2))
 (segment (start 117.729 95.316) (end 114.808 95.316) (width 0.25) (layer "F.Cu") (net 2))
 (segment (start 140.3091 99.822) (end 141.0429 99.0882) (width 0.25) (layer "F.Cu") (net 2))
 (segment (start 119.3799 94.742) (end 135.5631 94.742) (width 0.25) (layer "F.Cu") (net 2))
 (segment (start 110.91 99.214) (end 113.8611 96.2629) (width 0.25) (layer "F.Cu") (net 2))
 (segment (start 138.176 96.012) (end 141.0429 96.012) (width 0.25) (layer "F.Cu") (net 2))
 (segment (start 138.176 96.012) (end 136.8331 96.012) (width 0.25) (layer "F.Cu") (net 2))
 (segment (start 110.91 103.873) (end 110.91 100.584) (width 0.25) (layer "F.Cu") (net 2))
 (segment (start 123.6248 113.538) (end 137.3408 99.822) (width 0.25) (layer "F.Cu") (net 2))
 (segment (start 141.0429 99.0882) (end 141.0429 96.012) (width 0.25) (layer "F.Cu") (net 2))
 (segment (start 118.2675 95.316) (end 118.8059 95.316) (width 0.25) (layer "F.Cu") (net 2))
 (segment (start 117.5696 113.538) (end 117.1561 113.538) (width 0.25) (layer "F.Cu") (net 2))
 (segment (start 110.91 100.584) (end 110.91 99.214) (width 0.25) (layer "F.Cu") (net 2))
 (segment (start 112.141 109.728) (end 113.391 110.978) (width 0.25) (layer "F.Cu") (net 2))
 (segment (start 137.3408 99.822) (end 140.3091 99.822) (width 0.25) (layer "F.Cu") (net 2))
 (segment (start 135.5631 94.742) (end 136.8331 96.012) (width 0.25) (layer "F.Cu") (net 2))
 (segment (start 113.8611 96.2629) (end 114.808 96.2629) (width 0.25) (layer "F.Cu") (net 2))
 (segment (start 118.8059 95.316) (end 119.3799 94.742) (width 0.25) (layer "F.Cu") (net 2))
 (segment (start 114.808 95.316) (end 114.808 96.2629) (width 0.25) (layer "F.Cu") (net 2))
 (segment (start 118.2675 95.316) (end 117.729 95.316) (width 0.25) (layer "F.Cu") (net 2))
 (segment (start 117.983 113.538) (end 123.6248 113.538) (width 0.25) (layer "F.Cu") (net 2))
 (segment (start 113.391 111.728) (end 115.201 113.538) (width 0.25) (layer "F.Cu") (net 2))
 (segment (start 113.414 105.167) (end 113.414 105.7939) (width 0.25) (layer "F.Cu") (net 1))
 (segment (start 118.8059 97.216) (end 118.8885 97.2986) (width 0.25) (layer "F.Cu") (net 1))
 (segment (start 123.6071 97.2986) (end 124.3121 98.0036) (width 0.25) (layer "F.Cu") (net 1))
 (segment (start 136.8331 98.552) (end 124.3121 98.552) (width 0.25) (layer "F.Cu") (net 1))
 (segment (start 109.4022 108.978) (end 110.141 108.978) (width 0.25) (layer "F.Cu") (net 1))
 (segment (start 109.4022 108.978) (end 109.4022 108.2396) (width 0.25) (layer "F.Cu") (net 1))
 (segment (start 118.8885 97.2986) (end 123.6071 97.2986) (width 0.25) (layer "F.Cu") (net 1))
 (segment (start 124.3121 101.6477) (end 123.5978 102.362) (width 0.25) (layer "F.Cu") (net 1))
 (segment (start 124.3121 98.0036) (end 124.3121 98.552) (width 0.25) (layer "F.Cu") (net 1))
 (segment (start 109.9245 111.728) (end 109.4022 111.2057) (width 0.25) (layer "F.Cu") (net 1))
 (segment (start 114.041 105.167) (end 113.414 105.167) (width 0.25) (layer "F.Cu") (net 1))
 (segment (start 113.2268 105.9811) (end 113.414 105.7939) (width 0.25) (layer "F.Cu") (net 1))
 (segment (start 123.5978 102.362) (end 116.846 102.362) (width 0.25) (layer "F.Cu") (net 1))
 (segment (start 110.891 111.728) (end 109.9245 111.728) (width 0.25) (layer "F.Cu") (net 1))
 (segment (start 117.729 97.216) (end 114.808 97.216) (width 0.25) (layer "F.Cu") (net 1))
 (segment (start 117.729 97.216) (end 118.8059 97.216) (width 0.25) (layer "F.Cu") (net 1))
 (segment (start 109.4022 111.2057) (end 109.4022 108.978) (width 0.25) (layer "F.Cu") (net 1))
 (segment (start 111.6607 105.9811) (end 113.2268 105.9811) (width 0.25) (layer "F.Cu") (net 1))
 (segment (start 109.4022 108.2396) (end 111.6607 105.9811) (width 0.25) (layer "F.Cu") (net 1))
 (segment (start 116.846 102.362) (end 114.041 105.167) (width 0.25) (layer "F.Cu") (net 1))
 (segment (start 124.3121 98.552) (end 124.3121 101.6477) (width 0.25) (layer "F.Cu") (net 1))
 (segment (start 138.176 98.552) (end 136.8331 98.552) (width 0.25) (layer "F.Cu") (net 1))
 (segment (start 112.564 103.367) (end 112.564 101.4569) (width 0.25) (layer "F.Cu") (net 16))
 (segment (start 112.61 100.584) (end 112.61 101.4109) (width 0.25) (layer "F.Cu") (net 16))
 (segment (start 112.564 101.4569) (end 112.61 101.4109) (width 0.25) (layer "F.Cu") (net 16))
 (segment (start 115.7961 110.478) (end 117.1561 111.838) (width 0.25) (layer "F.Cu") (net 25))
 (segment (start 117.983 111.838) (end 117.1561 111.838) (width 0.25) (layer "F.Cu") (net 25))
 (segment (start 114.141 110.478) (end 115.7961 110.478) (width 0.25) (layer "F.Cu") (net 25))
 (segment (start 117.1051 108.978) (end 117.2831 108.8) (width 0.25) (layer "F.Cu") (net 28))
 (segment (start 118.11 108.8) (end 117.2831 108.8) (width 0.25) (layer "F.Cu") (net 28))
 (segment (start 114.141 108.978) (end 117.1051 108.978) (width 0.25) (layer "F.Cu") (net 28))
 (segment (start 114.141 108.478) (end 114.141 107.4509) (width 0.25) (layer "F.Cu") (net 3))
 (segment (start 117.006 103.759) (end 117.006 104.5859) (width 0.25) (layer "F.Cu") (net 3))
 (segment (start 114.141 107.4509) (end 117.006 104.5859) (width 0.25) (layer "F.Cu") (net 3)))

